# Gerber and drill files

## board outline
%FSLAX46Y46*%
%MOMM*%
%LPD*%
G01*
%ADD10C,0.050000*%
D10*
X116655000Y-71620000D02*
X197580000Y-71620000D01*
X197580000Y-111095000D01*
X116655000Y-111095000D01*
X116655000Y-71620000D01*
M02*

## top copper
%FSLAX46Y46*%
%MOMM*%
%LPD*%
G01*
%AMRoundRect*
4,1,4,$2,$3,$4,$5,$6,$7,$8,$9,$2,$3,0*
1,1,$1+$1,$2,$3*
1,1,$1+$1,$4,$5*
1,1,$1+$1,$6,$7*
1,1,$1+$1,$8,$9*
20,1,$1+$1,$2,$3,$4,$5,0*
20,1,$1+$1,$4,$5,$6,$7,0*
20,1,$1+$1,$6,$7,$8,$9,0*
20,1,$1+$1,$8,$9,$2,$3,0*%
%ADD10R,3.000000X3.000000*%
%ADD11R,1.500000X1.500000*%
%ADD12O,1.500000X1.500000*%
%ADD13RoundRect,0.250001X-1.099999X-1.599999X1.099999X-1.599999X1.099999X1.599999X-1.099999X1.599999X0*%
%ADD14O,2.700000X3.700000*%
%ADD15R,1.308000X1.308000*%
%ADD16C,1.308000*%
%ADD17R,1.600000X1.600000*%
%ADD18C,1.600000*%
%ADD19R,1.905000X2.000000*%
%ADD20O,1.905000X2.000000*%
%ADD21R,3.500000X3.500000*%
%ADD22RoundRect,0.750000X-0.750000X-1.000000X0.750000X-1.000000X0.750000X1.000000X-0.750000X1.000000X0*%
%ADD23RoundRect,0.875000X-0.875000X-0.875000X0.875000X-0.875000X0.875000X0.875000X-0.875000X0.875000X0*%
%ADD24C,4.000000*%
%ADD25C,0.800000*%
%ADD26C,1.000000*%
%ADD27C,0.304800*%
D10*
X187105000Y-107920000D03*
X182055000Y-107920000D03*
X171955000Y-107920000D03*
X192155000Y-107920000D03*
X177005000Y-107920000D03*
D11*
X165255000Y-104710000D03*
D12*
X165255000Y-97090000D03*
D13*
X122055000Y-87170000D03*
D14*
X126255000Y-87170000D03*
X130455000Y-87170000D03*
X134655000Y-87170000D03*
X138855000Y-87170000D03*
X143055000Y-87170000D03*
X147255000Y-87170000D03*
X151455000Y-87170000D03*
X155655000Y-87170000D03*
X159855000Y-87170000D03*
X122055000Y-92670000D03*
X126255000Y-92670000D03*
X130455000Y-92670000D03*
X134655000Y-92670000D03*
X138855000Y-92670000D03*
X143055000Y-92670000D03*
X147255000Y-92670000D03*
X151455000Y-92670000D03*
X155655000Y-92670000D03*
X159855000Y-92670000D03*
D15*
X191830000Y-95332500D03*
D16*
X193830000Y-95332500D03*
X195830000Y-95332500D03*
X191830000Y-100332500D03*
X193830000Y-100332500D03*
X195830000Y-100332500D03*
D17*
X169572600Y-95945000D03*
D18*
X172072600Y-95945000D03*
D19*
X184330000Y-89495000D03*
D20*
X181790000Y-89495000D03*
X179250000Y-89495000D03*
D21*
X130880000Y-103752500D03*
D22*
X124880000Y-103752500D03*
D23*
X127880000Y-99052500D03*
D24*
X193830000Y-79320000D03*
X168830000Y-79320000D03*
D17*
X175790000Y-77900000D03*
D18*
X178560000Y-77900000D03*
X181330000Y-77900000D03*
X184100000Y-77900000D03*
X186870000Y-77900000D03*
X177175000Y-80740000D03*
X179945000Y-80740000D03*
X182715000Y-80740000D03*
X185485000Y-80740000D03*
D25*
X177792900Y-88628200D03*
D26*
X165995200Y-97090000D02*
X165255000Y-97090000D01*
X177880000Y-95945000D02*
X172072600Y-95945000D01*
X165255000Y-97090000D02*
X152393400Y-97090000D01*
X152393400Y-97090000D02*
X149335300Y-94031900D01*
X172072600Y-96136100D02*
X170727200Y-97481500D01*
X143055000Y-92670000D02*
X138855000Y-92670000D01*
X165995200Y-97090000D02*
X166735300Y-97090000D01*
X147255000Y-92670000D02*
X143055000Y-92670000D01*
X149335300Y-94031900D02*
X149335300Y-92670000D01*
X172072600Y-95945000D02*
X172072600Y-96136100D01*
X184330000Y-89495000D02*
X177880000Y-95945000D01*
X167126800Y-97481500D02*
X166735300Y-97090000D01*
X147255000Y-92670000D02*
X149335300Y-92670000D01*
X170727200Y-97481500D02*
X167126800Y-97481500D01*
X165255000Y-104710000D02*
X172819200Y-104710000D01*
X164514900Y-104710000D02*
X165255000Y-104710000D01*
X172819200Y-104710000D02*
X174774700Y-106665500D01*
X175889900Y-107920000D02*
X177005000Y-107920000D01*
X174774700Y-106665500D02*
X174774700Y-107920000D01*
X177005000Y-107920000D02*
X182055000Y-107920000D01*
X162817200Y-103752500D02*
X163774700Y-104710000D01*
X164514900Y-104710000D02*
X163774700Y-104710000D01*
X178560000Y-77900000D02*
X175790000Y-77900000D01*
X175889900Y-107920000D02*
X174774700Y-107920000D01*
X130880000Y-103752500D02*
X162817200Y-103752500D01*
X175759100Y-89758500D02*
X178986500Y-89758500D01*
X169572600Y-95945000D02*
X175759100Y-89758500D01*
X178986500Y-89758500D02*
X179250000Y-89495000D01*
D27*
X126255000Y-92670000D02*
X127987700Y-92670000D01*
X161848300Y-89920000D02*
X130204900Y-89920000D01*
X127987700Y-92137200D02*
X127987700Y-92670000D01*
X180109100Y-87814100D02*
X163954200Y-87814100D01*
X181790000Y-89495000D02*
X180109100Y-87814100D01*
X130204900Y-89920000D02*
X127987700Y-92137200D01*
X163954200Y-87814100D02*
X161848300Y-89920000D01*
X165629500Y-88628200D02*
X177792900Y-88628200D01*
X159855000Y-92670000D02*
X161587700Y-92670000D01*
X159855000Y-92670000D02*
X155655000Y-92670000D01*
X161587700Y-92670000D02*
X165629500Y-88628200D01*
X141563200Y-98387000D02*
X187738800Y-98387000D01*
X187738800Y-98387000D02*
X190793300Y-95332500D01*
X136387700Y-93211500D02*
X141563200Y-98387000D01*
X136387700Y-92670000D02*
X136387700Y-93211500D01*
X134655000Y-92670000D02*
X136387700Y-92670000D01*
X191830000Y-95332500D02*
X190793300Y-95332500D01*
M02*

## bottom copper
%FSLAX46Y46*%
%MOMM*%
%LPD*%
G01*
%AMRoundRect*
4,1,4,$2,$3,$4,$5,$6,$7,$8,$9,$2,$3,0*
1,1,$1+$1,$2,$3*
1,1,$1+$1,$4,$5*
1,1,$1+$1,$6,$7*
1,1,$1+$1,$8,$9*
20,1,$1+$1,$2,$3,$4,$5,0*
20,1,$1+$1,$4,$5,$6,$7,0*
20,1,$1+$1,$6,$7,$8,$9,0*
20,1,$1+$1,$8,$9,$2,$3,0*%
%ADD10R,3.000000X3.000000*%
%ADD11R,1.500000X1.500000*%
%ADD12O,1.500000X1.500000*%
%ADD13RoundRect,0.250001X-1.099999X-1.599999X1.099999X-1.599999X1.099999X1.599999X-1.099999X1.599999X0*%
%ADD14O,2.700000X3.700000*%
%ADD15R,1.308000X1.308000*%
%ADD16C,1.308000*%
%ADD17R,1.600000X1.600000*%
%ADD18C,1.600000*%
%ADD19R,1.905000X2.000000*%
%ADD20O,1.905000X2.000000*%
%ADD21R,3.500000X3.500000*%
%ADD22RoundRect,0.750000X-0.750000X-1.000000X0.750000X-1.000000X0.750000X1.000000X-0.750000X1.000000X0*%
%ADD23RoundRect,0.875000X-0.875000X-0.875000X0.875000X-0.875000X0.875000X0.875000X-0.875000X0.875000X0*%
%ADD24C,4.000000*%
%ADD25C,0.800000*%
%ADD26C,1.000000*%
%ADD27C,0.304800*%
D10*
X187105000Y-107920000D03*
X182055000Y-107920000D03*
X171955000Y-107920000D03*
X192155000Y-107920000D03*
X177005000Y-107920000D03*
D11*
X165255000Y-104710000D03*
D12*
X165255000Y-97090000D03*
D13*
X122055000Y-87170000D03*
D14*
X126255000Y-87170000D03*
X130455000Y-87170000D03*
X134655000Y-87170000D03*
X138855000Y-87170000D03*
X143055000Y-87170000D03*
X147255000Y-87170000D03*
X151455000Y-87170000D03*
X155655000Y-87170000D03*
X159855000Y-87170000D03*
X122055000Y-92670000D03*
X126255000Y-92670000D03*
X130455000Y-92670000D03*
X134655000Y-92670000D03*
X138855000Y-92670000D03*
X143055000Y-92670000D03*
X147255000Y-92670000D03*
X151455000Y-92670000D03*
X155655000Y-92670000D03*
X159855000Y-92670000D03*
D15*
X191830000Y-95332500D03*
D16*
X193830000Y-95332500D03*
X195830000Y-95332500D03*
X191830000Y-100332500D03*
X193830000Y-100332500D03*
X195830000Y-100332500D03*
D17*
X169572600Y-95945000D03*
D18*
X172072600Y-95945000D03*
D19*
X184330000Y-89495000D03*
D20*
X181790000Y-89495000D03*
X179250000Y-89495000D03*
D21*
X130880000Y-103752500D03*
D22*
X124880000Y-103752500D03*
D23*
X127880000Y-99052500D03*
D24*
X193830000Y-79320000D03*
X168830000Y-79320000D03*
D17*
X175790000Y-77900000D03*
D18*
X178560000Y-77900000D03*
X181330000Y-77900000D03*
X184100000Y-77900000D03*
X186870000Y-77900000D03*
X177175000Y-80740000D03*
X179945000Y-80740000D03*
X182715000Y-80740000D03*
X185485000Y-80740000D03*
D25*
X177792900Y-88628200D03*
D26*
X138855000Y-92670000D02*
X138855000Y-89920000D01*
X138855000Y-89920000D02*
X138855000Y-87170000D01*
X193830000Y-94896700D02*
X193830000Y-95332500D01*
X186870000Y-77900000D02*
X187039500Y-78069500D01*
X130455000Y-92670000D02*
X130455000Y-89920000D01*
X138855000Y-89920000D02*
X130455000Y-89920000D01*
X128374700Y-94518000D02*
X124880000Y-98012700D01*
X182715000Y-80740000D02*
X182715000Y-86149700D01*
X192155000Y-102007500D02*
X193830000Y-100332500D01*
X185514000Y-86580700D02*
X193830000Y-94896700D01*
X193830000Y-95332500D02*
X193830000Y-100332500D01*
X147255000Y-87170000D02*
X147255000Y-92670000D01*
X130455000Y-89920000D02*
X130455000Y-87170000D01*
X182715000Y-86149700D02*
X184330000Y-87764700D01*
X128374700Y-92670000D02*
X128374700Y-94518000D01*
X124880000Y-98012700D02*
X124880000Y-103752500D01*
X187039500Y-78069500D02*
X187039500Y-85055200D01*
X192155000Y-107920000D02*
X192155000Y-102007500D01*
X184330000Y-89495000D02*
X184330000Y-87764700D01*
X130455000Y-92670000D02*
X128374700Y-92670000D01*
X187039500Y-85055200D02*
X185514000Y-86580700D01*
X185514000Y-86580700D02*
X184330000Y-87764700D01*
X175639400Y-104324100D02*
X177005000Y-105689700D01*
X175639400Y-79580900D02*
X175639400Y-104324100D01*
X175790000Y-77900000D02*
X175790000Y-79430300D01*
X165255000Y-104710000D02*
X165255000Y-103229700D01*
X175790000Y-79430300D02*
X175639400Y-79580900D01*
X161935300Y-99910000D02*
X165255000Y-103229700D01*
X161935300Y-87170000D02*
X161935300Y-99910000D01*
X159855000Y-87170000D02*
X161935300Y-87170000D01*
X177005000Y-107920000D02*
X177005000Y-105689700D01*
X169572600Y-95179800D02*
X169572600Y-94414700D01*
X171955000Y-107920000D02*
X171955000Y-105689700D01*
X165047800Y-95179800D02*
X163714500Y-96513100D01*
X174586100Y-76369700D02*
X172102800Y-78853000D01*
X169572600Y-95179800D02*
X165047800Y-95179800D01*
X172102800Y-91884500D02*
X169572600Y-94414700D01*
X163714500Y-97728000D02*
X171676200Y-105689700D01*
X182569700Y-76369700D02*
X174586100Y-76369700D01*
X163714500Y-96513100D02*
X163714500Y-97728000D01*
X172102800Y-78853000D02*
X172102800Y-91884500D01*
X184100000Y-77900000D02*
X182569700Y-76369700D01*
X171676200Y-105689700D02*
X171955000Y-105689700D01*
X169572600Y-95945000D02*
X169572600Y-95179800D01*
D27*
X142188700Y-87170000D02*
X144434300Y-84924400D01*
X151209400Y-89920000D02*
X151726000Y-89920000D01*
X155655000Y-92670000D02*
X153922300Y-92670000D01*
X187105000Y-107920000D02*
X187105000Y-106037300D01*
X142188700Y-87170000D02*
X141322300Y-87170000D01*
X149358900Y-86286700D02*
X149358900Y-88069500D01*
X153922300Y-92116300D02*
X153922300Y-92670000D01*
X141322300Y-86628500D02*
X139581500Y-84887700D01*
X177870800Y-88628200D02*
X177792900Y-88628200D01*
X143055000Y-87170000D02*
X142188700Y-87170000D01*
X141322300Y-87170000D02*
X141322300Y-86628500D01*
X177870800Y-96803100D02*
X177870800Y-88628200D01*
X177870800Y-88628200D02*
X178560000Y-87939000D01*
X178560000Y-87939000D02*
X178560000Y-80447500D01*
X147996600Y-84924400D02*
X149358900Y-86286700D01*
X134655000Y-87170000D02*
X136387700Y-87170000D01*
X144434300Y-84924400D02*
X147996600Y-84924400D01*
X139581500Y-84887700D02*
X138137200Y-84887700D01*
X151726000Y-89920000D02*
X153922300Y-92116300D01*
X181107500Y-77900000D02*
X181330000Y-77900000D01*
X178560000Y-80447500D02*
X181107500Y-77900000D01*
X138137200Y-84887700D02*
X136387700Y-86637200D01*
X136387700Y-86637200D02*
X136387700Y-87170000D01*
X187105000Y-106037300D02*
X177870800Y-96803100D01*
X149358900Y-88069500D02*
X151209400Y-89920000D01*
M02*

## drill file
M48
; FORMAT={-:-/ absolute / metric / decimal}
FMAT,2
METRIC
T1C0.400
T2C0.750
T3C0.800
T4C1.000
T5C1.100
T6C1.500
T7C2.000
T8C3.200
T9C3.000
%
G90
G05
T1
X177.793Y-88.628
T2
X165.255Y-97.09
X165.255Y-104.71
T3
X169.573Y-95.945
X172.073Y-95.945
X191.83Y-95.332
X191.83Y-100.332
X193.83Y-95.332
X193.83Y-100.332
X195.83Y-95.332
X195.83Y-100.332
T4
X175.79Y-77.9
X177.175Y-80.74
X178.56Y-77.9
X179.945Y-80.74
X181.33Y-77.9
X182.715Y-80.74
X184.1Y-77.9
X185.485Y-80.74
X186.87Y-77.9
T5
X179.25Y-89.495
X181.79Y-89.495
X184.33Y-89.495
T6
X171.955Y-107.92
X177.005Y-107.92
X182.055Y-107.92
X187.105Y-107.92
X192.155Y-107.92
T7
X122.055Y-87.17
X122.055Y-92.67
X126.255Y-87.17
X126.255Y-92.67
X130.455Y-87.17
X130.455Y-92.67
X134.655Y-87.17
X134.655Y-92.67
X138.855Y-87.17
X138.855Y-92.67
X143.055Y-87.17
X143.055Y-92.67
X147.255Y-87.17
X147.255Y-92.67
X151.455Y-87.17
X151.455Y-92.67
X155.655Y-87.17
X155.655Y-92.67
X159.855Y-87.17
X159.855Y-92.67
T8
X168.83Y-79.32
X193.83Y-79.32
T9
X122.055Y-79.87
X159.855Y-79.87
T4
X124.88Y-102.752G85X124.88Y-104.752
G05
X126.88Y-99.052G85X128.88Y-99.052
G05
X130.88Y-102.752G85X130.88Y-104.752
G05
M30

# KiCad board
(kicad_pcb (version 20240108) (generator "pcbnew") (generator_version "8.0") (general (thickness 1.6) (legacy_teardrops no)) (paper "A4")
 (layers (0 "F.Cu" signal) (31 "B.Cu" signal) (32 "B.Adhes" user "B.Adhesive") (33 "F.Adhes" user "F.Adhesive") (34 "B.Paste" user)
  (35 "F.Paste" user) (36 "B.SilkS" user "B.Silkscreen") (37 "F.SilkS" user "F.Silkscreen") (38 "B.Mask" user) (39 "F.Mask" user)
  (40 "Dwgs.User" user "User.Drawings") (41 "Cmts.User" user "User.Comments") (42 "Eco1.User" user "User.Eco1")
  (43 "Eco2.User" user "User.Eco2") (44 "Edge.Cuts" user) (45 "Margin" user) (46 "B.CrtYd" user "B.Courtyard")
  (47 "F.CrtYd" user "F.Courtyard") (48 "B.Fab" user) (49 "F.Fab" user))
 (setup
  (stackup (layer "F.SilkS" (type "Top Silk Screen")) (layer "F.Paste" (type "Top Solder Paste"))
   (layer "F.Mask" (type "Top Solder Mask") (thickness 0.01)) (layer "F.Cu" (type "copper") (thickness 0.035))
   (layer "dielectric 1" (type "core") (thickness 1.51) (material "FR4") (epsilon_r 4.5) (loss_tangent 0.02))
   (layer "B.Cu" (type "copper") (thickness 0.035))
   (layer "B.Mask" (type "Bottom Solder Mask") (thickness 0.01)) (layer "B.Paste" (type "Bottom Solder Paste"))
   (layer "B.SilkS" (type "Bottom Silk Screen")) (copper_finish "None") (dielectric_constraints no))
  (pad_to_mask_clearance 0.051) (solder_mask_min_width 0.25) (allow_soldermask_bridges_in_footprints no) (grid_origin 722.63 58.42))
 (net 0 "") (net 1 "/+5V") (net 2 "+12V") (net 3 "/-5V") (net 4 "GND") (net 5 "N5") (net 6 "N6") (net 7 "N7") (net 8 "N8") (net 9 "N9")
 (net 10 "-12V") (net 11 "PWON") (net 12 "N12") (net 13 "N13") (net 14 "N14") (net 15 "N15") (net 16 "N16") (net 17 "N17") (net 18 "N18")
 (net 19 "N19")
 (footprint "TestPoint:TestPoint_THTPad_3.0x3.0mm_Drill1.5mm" (layer "F.Cu") (at 187.105 107.92)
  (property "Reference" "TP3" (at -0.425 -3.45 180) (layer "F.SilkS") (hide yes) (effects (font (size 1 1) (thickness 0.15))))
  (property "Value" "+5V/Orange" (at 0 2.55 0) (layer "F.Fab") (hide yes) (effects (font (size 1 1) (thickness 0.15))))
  (pad "1" thru_hole rect (at 0 0) (size 3 3) (drill 1.5) (layers "*.Cu" "*.Mask") (remove_unused_layers no) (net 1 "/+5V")))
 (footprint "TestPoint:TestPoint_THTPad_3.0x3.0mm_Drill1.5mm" (layer "F.Cu") (at 182.055 107.92)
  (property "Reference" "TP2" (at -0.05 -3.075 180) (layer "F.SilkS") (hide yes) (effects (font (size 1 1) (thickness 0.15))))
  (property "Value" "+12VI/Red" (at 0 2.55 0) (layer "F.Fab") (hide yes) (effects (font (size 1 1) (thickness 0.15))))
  (pad "1" thru_hole rect (at 0 0) (size 3 3) (drill 1.5) (layers "*.Cu" "*.Mask") (remove_unused_layers no) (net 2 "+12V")))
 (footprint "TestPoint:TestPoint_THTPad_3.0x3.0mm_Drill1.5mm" (layer "F.Cu") (at 171.955 107.92)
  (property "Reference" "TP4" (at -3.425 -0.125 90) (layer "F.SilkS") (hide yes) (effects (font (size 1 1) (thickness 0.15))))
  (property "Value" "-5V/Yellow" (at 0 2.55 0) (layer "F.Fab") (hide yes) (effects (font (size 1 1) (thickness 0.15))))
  (pad "1" thru_hole rect (at 0 0) (size 3 3) (drill 1.5) (layers "*.Cu" "*.Mask") (remove_unused_layers no) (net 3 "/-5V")))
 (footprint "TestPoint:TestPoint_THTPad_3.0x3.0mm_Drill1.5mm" (layer "F.Cu") (at 192.155 107.92)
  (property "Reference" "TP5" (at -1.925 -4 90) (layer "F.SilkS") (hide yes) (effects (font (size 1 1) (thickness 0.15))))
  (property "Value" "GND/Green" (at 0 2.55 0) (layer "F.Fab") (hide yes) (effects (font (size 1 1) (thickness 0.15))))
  (pad "1" thru_hole rect (at 0 0) (size 3 3) (drill 1.5) (layers "*.Cu" "*.Mask") (remove_unused_layers no) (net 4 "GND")))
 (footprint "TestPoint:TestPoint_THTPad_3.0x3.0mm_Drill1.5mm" (layer "F.Cu") (at 177.005 107.92)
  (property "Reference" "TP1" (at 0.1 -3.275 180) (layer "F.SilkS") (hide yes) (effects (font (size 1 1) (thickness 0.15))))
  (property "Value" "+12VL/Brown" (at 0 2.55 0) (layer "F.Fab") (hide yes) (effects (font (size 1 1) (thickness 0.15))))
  (pad "1" thru_hole rect (at 0 0) (size 3 3) (drill 1.5) (layers "*.Cu" "*.Mask") (remove_unused_layers no) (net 2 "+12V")))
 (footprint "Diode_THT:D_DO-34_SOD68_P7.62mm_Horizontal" (layer "F.Cu") (at 165.255 104.71 90)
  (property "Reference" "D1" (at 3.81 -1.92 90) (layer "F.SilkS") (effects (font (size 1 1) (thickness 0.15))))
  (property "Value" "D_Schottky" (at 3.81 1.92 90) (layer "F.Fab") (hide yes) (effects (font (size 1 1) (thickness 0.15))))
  (pad "1" thru_hole rect (at 0 0 90) (size 1.5 1.5) (drill 0.75) (layers "*.Cu" "*.Mask") (remove_unused_layers no) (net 2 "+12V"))
  (pad "2" thru_hole oval (at 7.62 0 90) (size 1.5 1.5) (drill 0.75) (layers "*.Cu" "*.Mask") (remove_unused_layers no) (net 4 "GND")))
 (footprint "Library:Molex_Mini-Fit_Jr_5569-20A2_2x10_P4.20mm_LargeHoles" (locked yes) (layer "F.Cu") (at 122.055 87.17)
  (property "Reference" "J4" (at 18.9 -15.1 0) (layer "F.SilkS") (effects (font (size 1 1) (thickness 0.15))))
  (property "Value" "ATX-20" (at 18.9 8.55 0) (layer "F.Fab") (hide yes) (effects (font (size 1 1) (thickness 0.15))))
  (pad "" np_thru_hole circle (at 0 -7.3) (size 3 3) (drill 3) (layers "*.Cu" "*.Mask"))
  (pad "" np_thru_hole circle (at 37.8 -7.3) (size 3 3) (drill 3) (layers "*.Cu" "*.Mask"))
  (pad "1" thru_hole roundrect (at 0 0) (size 2.7 3.7) (drill 2) (layers "*.Cu" "*.Mask") (remove_unused_layers no)
   (roundrect_rratio 0.092593) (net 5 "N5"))
  (pad "2" thru_hole oval (at 4.2 0) (size 2.7 3.7) (drill 2) (layers "*.Cu" "*.Mask") (remove_unused_layers no) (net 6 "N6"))
  (pad "3" thru_hole oval (at 8.4 0) (size 2.7 3.7) (drill 2) (layers "*.Cu" "*.Mask") (remove_unused_layers no) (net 4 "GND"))
  (pad "4" thru_hole oval (at 12.6 0) (size 2.7 3.7) (drill 2) (layers "*.Cu" "*.Mask") (remove_unused_layers no) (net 1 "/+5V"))
  (pad "5" thru_hole oval (at 16.8 0) (size 2.7 3.7) (drill 2) (layers "*.Cu" "*.Mask") (remove_unused_layers no) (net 4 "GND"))
  (pad "6" thru_hole oval (at 21 0) (size 2.7 3.7) (drill 2) (layers "*.Cu" "*.Mask") (remove_unused_layers no) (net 1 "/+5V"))
  (pad "7" thru_hole oval (at 25.2 0) (size 2.7 3.7) (drill 2) (layers "*.Cu" "*.Mask") (remove_unused_layers no) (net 4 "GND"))
  (pad "8" thru_hole oval (at 29.4 0) (size 2.7 3.7) (drill 2) (layers "*.Cu" "*.Mask") (remove_unused_layers no) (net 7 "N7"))
  (pad "9" thru_hole oval (at 33.6 0) (size 2.7 3.7) (drill 2) (layers "*.Cu" "*.Mask") (remove_unused_layers no) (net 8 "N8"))
  (pad "10" thru_hole oval (at 37.8 0) (size 2.7 3.7) (drill 2) (layers "*.Cu" "*.Mask") (remove_unused_layers no) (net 2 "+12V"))
  (pad "11" thru_hole oval (at 0 5.5) (size 2.7 3.7) (drill 2) (layers "*.Cu" "*.Mask") (remove_unused_layers no) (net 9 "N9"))
  (pad "12" thru_hole oval (at 4.2 5.5) (size 2.7 3.7) (drill 2) (layers "*.Cu" "*.Mask") (remove_unused_layers no) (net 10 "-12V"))
  (pad "13" thru_hole oval (at 8.4 5.5) (size 2.7 3.7) (drill 2) (layers "*.Cu" "*.Mask") (remove_unused_layers no) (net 4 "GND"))
  (pad "14" thru_hole oval (at 12.6 5.5) (size 2.7 3.7) (drill 2) (layers "*.Cu" "*.Mask") (remove_unused_layers no) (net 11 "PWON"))
  (pad "15" thru_hole oval (at 16.8 5.5) (size 2.7 3.7) (drill 2) (layers "*.Cu" "*.Mask") (remove_unused_layers no) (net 4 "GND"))
  (pad "16" thru_hole oval (at 21 5.5) (size 2.7 3.7) (drill 2) (layers "*.Cu" "*.Mask") (remove_unused_layers no) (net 4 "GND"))
  (pad "17" thru_hole oval (at 25.2 5.5) (size 2.7 3.7) (drill 2) (layers "*.Cu" "*.Mask") (remove_unused_layers no) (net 4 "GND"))
  (pad "18" thru_hole oval (at 29.4 5.5) (size 2.7 3.7) (drill 2) (layers "*.Cu" "*.Mask") (remove_unused_layers no) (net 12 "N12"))
  (pad "19" thru_hole oval (at 33.6 5.5) (size 2.7 3.7) (drill 2) (layers "*.Cu" "*.Mask") (remove_unused_layers no) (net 1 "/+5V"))
  (pad "20" thru_hole oval (at 37.8 5.5) (size 2.7 3.7) (drill 2) (layers "*.Cu" "*.Mask") (remove_unused_layers no) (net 1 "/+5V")))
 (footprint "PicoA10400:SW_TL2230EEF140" (layer "F.Cu") (at 193.83 97.8325)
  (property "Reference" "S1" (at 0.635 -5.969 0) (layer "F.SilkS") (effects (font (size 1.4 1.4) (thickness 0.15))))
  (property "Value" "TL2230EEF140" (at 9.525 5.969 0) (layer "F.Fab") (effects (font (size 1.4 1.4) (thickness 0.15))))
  (pad "1" thru_hole rect (at -2 -2.5) (size 1.308 1.308) (drill 0.8) (layers "*.Cu" "*.Mask") (remove_unused_layers no) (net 11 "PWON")
   (solder_mask_margin 0.102))
  (pad "2" thru_hole circle (at 0 -2.5) (size 1.308 1.308) (drill 0.8) (layers "*.Cu" "*.Mask") (remove_unused_layers no) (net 4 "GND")
   (solder_mask_margin 0.102))
  (pad "3" thru_hole circle (at 2 -2.5) (size 1.308 1.308) (drill 0.8) (layers "*.Cu" "*.Mask") (remove_unused_layers no) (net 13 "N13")
   (solder_mask_margin 0.102))
  (pad "4" thru_hole circle (at -2 2.5) (size 1.308 1.308) (drill 0.8) (layers "*.Cu" "*.Mask") (remove_unused_layers no) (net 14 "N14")
   (solder_mask_margin 0.102))
  (pad "5" thru_hole circle (at 0 2.5) (size 1.308 1.308) (drill 0.8) (layers "*.Cu" "*.Mask") (remove_unused_layers no) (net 4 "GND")
   (solder_mask_margin 0.102))
  (pad "6" thru_hole circle (at 2 2.5) (size 1.308 1.308) (drill 0.8) (layers "*.Cu" "*.Mask") (remove_unused_layers no) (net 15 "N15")
   (solder_mask_margin 0.102)))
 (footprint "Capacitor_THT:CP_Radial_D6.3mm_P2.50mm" (layer "F.Cu") (at 169.5726 95.945)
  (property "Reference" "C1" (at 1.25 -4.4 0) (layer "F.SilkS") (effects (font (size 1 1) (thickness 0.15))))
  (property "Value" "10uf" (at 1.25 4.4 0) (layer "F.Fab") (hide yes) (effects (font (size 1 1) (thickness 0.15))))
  (pad "1" thru_hole rect (at 0 0) (size 1.6 1.6) (drill 0.8) (layers "*.Cu" "*.Mask") (remove_unused_layers no) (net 3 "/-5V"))
  (pad "2" thru_hole circle (at 2.5 0) (size 1.6 1.6) (drill 0.8) (layers "*.Cu" "*.Mask") (remove_unused_layers no) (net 4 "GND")))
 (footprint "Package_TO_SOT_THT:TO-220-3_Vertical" (layer "F.Cu") (at 184.33 89.495 180)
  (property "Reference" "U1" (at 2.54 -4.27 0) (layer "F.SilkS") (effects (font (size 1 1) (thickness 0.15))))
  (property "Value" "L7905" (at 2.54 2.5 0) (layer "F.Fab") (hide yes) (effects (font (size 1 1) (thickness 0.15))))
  (pad "1" thru_hole rect (at 0 0 180) (size 1.905 2) (drill 1.1) (layers "*.Cu" "*.Mask") (remove_unused_layers no) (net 4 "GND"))
  (pad "2" thru_hole oval (at 2.54 0 180) (size 1.905 2) (drill 1.1) (layers "*.Cu" "*.Mask") (remove_unused_layers no) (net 10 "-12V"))
  (pad "3" thru_hole oval (at 5.08 0 180) (size 1.905 2) (drill 1.1) (layers "*.Cu" "*.Mask") (remove_unused_layers no) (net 3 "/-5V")))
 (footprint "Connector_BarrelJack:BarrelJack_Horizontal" (layer "B.Cu") (at 130.88 103.7525)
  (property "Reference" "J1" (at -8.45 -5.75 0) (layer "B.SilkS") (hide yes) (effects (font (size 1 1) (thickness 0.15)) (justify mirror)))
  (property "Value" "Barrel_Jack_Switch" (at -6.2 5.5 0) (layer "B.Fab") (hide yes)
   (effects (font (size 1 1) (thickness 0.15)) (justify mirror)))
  (pad "1" thru_hole rect (at 0 0) (size 3.5 3.5) (drill oval 1 3) (layers "*.Cu" "*.Mask") (remove_unused_layers no) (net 2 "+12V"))
  (pad "2" thru_hole roundrect (at -6 0) (size 3 3.5) (drill oval 1 3) (layers "*.Cu" "*.Mask") (remove_unused_layers no)
   (roundrect_rratio 0.25) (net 4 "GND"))
  (pad "3" thru_hole roundrect (at -3 -4.7) (size 3.5 3.5) (drill oval 3 1) (layers "*.Cu" "*.Mask") (remove_unused_layers no)
   (roundrect_rratio 0.25) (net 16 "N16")))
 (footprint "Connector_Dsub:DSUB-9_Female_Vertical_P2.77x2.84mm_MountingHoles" (layer "B.Cu") (at 175.79 77.9 180)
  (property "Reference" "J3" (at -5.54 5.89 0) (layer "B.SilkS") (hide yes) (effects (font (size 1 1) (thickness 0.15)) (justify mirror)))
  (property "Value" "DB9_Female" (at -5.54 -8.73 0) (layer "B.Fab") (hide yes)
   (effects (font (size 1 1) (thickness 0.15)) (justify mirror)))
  (pad "0" thru_hole circle (at -18.04 -1.42 180) (size 4 4) (drill 3.2) (layers "*.Cu" "*.Mask") (remove_unused_layers no))
  (pad "0" thru_hole circle (at 6.96 -1.42 180) (size 4 4) (drill 3.2) (layers "*.Cu" "*.Mask") (remove_unused_layers no))
  (pad "1" thru_hole rect (at 0 0 180) (size 1.6 1.6) (drill 1) (layers "*.Cu" "*.Mask") (remove_unused_layers no) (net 2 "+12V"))
  (pad "2" thru_hole circle (at -2.77 0 180) (size 1.6 1.6) (drill 1) (layers "*.Cu" "*.Mask") (remove_unused_layers no) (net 2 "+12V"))
  (pad "3" thru_hole circle (at -5.54 0 180) (size 1.6 1.6) (drill 1) (layers "*.Cu" "*.Mask") (remove_unused_layers no) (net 1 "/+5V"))
  (pad "4" thru_hole circle (at -8.31 0 180) (size 1.6 1.6) (drill 1) (layers "*.Cu" "*.Mask") (remove_unused_layers no) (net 3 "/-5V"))
  (pad "5" thru_hole circle (at -11.08 0 180) (size 1.6 1.6) (drill 1) (layers "*.Cu" "*.Mask") (remove_unused_layers no) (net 4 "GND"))
  (pad "6" thru_hole circle (at -1.385 -2.84 180) (size 1.6 1.6) (drill 1) (layers "*.Cu" "*.Mask") (remove_unused_layers no) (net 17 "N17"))
  (pad "7" thru_hole circle (at -4.155 -2.84 180) (size 1.6 1.6) (drill 1) (layers "*.Cu" "*.Mask") (remove_unused_layers no) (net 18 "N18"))
  (pad "8" thru_hole circle (at -6.925 -2.84 180) (size 1.6 1.6) (drill 1) (layers "*.Cu" "*.Mask") (remove_unused_layers no) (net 4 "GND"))
  (pad "9" thru_hole circle (at -9.695 -2.84 180) (size 1.6 1.6) (drill 1) (layers "*.Cu" "*.Mask") (remove_unused_layers no) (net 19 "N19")))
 (gr_rect (start 116.655 71.62) (end 197.58 111.095) (stroke (width 0.05) (type default)) (fill none) (layer "Edge.Cuts"))
 (segment (start 165.9952 97.09) (end 165.255 97.09) (width 1) (layer "F.Cu") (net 4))
 (segment (start 177.88 95.945) (end 172.0726 95.945) (width 1) (layer "F.Cu") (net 4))
 (segment (start 165.255 97.09) (end 152.3934 97.09) (width 1) (layer "F.Cu") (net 4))
 (segment (start 152.3934 97.09) (end 149.3353 94.0319) (width 1) (layer "F.Cu") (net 4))
 (segment (start 172.0726 96.1361) (end 170.7272 97.4815) (width 1) (layer "F.Cu") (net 4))
 (segment (start 143.055 92.67) (end 138.855 92.67) (width 1) (layer "F.Cu") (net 4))
 (segment (start 165.9952 97.09) (end 166.7353 97.09) (width 1) (layer "F.Cu") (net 4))
 (segment (start 147.255 92.67) (end 143.055 92.67) (width 1) (layer "F.Cu") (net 4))
 (segment (start 149.3353 94.0319) (end 149.3353 92.67) (width 1) (layer "F.Cu") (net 4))
 (segment (start 172.0726 95.945) (end 172.0726 96.1361) (width 1) (layer "F.Cu") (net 4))
 (segment (start 184.33 89.495) (end 177.88 95.945) (width 1) (layer "F.Cu") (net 4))
 (segment (start 167.1268 97.4815) (end 166.7353 97.09) (width 1) (layer "F.Cu") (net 4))
 (segment (start 147.255 92.67) (end 149.3353 92.67) (width 1) (layer "F.Cu") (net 4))
 (segment (start 170.7272 97.4815) (end 167.1268 97.4815) (width 1) (layer "F.Cu") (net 4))
 (segment (start 138.855 92.67) (end 138.855 89.92) (width 1) (layer "B.Cu") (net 4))
 (segment (start 138.855 89.92) (end 138.855 87.17) (width 1) (layer "B.Cu") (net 4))
 (segment (start 193.83 94.8967) (end 193.83 95.3325) (width 1) (layer "B.Cu") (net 4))
 (segment (start 186.87 77.9) (end 187.0395 78.0695) (width 1) (layer "B.Cu") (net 4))
 (segment (start 130.455 92.67) (end 130.455 89.92) (width 1) (layer "B.Cu") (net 4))
 (segment (start 138.855 89.92) (end 130.455 89.92) (width 1) (layer "B.Cu") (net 4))
 (segment (start 128.3747 94.518) (end 124.88 98.0127) (width 1) (layer "B.Cu") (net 4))
 (segment (start 182.715 80.74) (end 182.715 86.1497) (width 1) (layer "B.Cu") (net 4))
 (segment (start 192.155 102.0075) (end 193.83 100.3325) (width 1) (layer "B.Cu") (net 4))
 (segment (start 185.514 86.5807) (end 193.83 94.8967) (width 1) (layer "B.Cu") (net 4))
 (segment (start 193.83 95.3325) (end 193.83 100.3325) (width 1) (layer "B.Cu") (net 4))
 (segment (start 147.255 87.17) (end 147.255 92.67) (width 1) (layer "B.Cu") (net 4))
 (segment (start 130.455 89.92) (end 130.455 87.17) (width 1) (layer "B.Cu") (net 4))
 (segment (start 182.715 86.1497) (end 184.33 87.7647) (width 1) (layer "B.Cu") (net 4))
 (segment (start 128.3747 92.67) (end 128.3747 94.518) (width 1) (layer "B.Cu") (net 4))
 (segment (start 124.88 98.0127) (end 124.88 103.7525) (width 1) (layer "B.Cu") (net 4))
 (segment (start 187.0395 78.0695) (end 187.0395 85.0552) (width 1) (layer "B.Cu") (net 4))
 (segment (start 192.155 107.92) (end 192.155 102.0075) (width 1) (layer "B.Cu") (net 4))
 (segment (start 184.33 89.495) (end 184.33 87.7647) (width 1) (layer "B.Cu") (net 4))
 (segment (start 130.455 92.67) (end 128.3747 92.67) (width 1) (layer "B.Cu") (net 4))
 (segment (start 187.0395 85.0552) (end 185.514 86.5807) (width 1) (layer "B.Cu") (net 4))
 (segment (start 185.514 86.5807) (end 184.33 87.7647) (width 1) (layer "B.Cu") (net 4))
 (segment (start 165.255 104.71) (end 172.8192 104.71) (width 1) (layer "F.Cu") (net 2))
 (segment (start 164.5149 104.71) (end 165.255 104.71) (width 1) (layer "F.Cu") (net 2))
 (segment (start 172.8192 104.71) (end 174.7747 106.6655) (width 1) (layer "F.Cu") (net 2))
 (segment (start 175.8899 107.92) (end 177.005 107.92) (width 1) (layer "F.Cu") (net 2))
 (segment (start 174.7747 106.6655) (end 174.7747 107.92) (width 1) (layer "F.Cu") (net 2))
 (segment (start 177.005 107.92) (end 182.055 107.92) (width 1) (layer "F.Cu") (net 2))
 (segment (start 162.8172 103.7525) (end 163.7747 104.71) (width 1) (layer "F.Cu") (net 2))
 (segment (start 164.5149 104.71) (end 163.7747 104.71) (width 1) (layer "F.Cu") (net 2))
 (segment (start 178.56 77.9) (end 175.79 77.9) (width 1) (layer "F.Cu") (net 2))
 (segment (start 175.8899 107.92) (end 174.7747 107.92) (width 1) (layer "F.Cu") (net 2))
 (segment (start 130.88 103.7525) (end 162.8172 103.7525) (width 1) (layer "F.Cu") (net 2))
 (segment (start 175.6394 104.3241) (end 177.005 105.6897) (width 1) (layer "B.Cu") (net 2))
 (segment (start 175.6394 79.5809) (end 175.6394 104.3241) (width 1) (layer "B.Cu") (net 2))
 (segment (start 175.79 77.9) (end 175.79 79.4303) (width 1) (layer "B.Cu") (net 2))
 (segment (start 165.255 104.71) (end 165.255 103.2297) (width 1) (layer "B.Cu") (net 2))
 (segment (start 175.79 79.4303) (end 175.6394 79.5809) (width 1) (layer "B.Cu") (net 2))
 (segment (start 161.9353 99.91) (end 165.255 103.2297) (width 1) (layer "B.Cu") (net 2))
 (segment (start 161.9353 87.17) (end 161.9353 99.91) (width 1) (layer "B.Cu") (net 2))
 (segment (start 159.855 87.17) (end 161.9353 87.17) (width 1) (layer "B.Cu") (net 2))
 (segment (start 177.005 107.92) (end 177.005 105.6897) (width 1) (layer "B.Cu") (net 2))
 (segment (start 175.7591 89.7585) (end 178.9865 89.7585) (width 1) (layer "F.Cu") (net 3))
 (segment (start 169.5726 95.945) (end 175.7591 89.7585) (width 1) (layer "F.Cu") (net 3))
 (segment (start 178.9865 89.7585) (end 179.25 89.495) (width 1) (layer "F.Cu") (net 3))
 (segment (start 169.5726 95.1798) (end 169.5726 94.4147) (width 1) (layer "B.Cu") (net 3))
 (segment (start 171.955 107.92) (end 171.955 105.6897) (width 1) (layer "B.Cu") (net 3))
 (segment (start 165.0478 95.1798) (end 163.7145 96.5131) (width 1) (layer "B.Cu") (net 3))
 (segment (start 174.5861 76.3697) (end 172.1028 78.853) (width 1) (layer "B.Cu") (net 3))
 (segment (start 169.5726 95.1798) (end 165.0478 95.1798) (width 1) (layer "B.Cu") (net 3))
 (segment (start 172.1028 91.8845) (end 169.5726 94.4147) (width 1) (layer "B.Cu") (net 3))
 (segment (start 163.7145 97.728) (end 171.6762 105.6897) (width 1) (layer "B.Cu") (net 3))
 (segment (start 182.5697 76.3697) (end 174.5861 76.3697) (width 1) (layer "B.Cu") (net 3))
 (segment (start 163.7145 96.5131) (end 163.7145 97.728) (width 1) (layer "B.Cu") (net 3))
 (segment (start 172.1028 78.853) (end 172.1028 91.8845) (width 1) (layer "B.Cu") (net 3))
 (segment (start 184.1 77.9) (end 182.5697 76.3697) (width 1) (layer "B.Cu") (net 3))
 (segment (start 171.6762 105.6897) (end 171.955 105.6897) (width 1) (layer "B.Cu") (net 3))
 (segment (start 169.5726 95.945) (end 169.5726 95.1798) (width 1) (layer "B.Cu") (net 3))
 (segment (start 126.255 92.67) (end 127.9877 92.67) (width 0.3048) (layer "F.Cu") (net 10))
 (segment (start 161.8483 89.92) (end 130.2049 89.92) (width 0.3048) (layer "F.Cu") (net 10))
 (segment (start 127.9877 92.1372) (end 127.9877 92.67) (width 0.3048) (layer "F.Cu") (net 10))
 (segment (start 180.1091 87.8141) (end 163.9542 87.8141) (width 0.3048) (layer "F.Cu") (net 10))
 (segment (start 181.79 89.495) (end 180.1091 87.8141) (width 0.3048) (layer "F.Cu") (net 10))
 (segment (start 130.2049 89.92) (end 127.9877 92.1372) (width 0.3048) (layer "F.Cu") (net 10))
 (segment (start 163.9542 87.8141) (end 161.8483 89.92) (width 0.3048) (layer "F.Cu") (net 10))
 (segment (start 165.6295 88.6282) (end 177.7929 88.6282) (width 0.3048) (layer "F.Cu") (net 1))
 (segment (start 159.855 92.67) (end 161.5877 92.67) (width 0.3048) (layer "F.Cu") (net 1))
 (segment (start 159.855 92.67) (end 155.655 92.67) (width 0.3048) (layer "F.Cu") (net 1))
 (segment (start 161.5877 92.67) (end 165.6295 88.6282) (width 0.3048) (layer "F.Cu") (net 1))
 (via (at 177.7929 88.6282) (size 0.8) (drill 0.4) (layers "F.Cu" "B.Cu") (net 1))
 (segment (start 142.1887 87.17) (end 144.4343 84.9244) (width 0.3048) (layer "B.Cu") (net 1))
 (segment (start 151.2094 89.92) (end 151.726 89.92) (width 0.3048) (layer "B.Cu") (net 1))
 (segment (start 155.655 92.67) (end 153.9223 92.67) (width 0.3048) (layer "B.Cu") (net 1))
 (segment (start 187.105 107.92) (end 187.105 106.0373) (width 0.3048) (layer "B.Cu") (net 1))
 (segment (start 142.1887 87.17) (end 141.3223 87.17) (width 0.3048) (layer "B.Cu") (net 1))
 (segment (start 149.3589 86.2867) (end 149.3589 88.0695) (width 0.3048) (layer "B.Cu") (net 1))
 (segment (start 153.9223 92.1163) (end 153.9223 92.67) (width 0.3048) (layer "B.Cu") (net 1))
 (segment (start 141.3223 86.6285) (end 139.5815 84.8877) (width 0.3048) (layer "B.Cu") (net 1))
 (segment (start 177.8708 88.6282) (end 177.7929 88.6282) (width 0.3048) (layer "B.Cu") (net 1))
 (segment (start 143.055 87.17) (end 142.1887 87.17) (width 0.3048) (layer "B.Cu") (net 1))
 (segment (start 141.3223 87.17) (end 141.3223 86.6285) (width 0.3048) (layer "B.Cu") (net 1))
 (segment (start 177.8708 96.8031) (end 177.8708 88.6282) (width 0.3048) (layer "B.Cu") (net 1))
 (segment (start 177.8708 88.6282) (end 178.56 87.939) (width 0.3048) (layer "B.Cu") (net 1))
 (segment (start 178.56 87.939) (end 178.56 80.4475) (width 0.3048) (layer "B.Cu") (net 1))
 (segment (start 147.9966 84.9244) (end 149.3589 86.2867) (width 0.3048) (layer "B.Cu") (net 1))
 (segment (start 134.655 87.17) (end 136.3877 87.17) (width 0.3048) (layer "B.Cu") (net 1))
 (segment (start 144.4343 84.9244) (end 147.9966 84.9244) (width 0.3048) (layer "B.Cu") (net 1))
 (segment (start 139.5815 84.8877) (end 138.1372 84.8877) (width 0.3048) (layer "B.Cu") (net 1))
 (segment (start 151.726 89.92) (end 153.9223 92.1163) (width 0.3048) (layer "B.Cu") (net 1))
 (segment (start 181.1075 77.9) (end 181.33 77.9) (width 0.3048) (layer "B.Cu") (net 1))
 (segment (start 178.56 80.4475) (end 181.1075 77.9) (width 0.3048) (layer "B.Cu") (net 1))
 (segment (start 138.1372 84.8877) (end 136.3877 86.6372) (width 0.3048) (layer "B.Cu") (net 1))
 (segment (start 136.3877 86.6372) (end 136.3877 87.17) (width 0.3048) (layer "B.Cu") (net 1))
 (segment (start 187.105 106.0373) (end 177.8708 96.8031) (width 0.3048) (layer "B.Cu") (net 1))
 (segment (start 149.3589 88.0695) (end 151.2094 89.92) (width 0.3048) (layer "B.Cu") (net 1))
 (segment (start 141.5632 98.387) (end 187.7388 98.387) (width 0.3048) (layer "F.Cu") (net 11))
 (segment (start 187.7388 98.387) (end 190.7933 95.3325) (width 0.3048) (layer "F.Cu") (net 11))
 (segment (start 136.3877 93.2115) (end 141.5632 98.387) (width 0.3048) (layer "F.Cu") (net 11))
 (segment (start 136.3877 92.67) (end 136.3877 93.2115) (width 0.3048) (layer "F.Cu") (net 11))
 (segment (start 134.655 92.67) (end 136.3877 92.67) (width 0.3048) (layer "F.Cu") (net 11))
 (segment (start 191.83 95.3325) (end 190.7933 95.3325) (width 0.3048) (layer "F.Cu") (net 11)))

